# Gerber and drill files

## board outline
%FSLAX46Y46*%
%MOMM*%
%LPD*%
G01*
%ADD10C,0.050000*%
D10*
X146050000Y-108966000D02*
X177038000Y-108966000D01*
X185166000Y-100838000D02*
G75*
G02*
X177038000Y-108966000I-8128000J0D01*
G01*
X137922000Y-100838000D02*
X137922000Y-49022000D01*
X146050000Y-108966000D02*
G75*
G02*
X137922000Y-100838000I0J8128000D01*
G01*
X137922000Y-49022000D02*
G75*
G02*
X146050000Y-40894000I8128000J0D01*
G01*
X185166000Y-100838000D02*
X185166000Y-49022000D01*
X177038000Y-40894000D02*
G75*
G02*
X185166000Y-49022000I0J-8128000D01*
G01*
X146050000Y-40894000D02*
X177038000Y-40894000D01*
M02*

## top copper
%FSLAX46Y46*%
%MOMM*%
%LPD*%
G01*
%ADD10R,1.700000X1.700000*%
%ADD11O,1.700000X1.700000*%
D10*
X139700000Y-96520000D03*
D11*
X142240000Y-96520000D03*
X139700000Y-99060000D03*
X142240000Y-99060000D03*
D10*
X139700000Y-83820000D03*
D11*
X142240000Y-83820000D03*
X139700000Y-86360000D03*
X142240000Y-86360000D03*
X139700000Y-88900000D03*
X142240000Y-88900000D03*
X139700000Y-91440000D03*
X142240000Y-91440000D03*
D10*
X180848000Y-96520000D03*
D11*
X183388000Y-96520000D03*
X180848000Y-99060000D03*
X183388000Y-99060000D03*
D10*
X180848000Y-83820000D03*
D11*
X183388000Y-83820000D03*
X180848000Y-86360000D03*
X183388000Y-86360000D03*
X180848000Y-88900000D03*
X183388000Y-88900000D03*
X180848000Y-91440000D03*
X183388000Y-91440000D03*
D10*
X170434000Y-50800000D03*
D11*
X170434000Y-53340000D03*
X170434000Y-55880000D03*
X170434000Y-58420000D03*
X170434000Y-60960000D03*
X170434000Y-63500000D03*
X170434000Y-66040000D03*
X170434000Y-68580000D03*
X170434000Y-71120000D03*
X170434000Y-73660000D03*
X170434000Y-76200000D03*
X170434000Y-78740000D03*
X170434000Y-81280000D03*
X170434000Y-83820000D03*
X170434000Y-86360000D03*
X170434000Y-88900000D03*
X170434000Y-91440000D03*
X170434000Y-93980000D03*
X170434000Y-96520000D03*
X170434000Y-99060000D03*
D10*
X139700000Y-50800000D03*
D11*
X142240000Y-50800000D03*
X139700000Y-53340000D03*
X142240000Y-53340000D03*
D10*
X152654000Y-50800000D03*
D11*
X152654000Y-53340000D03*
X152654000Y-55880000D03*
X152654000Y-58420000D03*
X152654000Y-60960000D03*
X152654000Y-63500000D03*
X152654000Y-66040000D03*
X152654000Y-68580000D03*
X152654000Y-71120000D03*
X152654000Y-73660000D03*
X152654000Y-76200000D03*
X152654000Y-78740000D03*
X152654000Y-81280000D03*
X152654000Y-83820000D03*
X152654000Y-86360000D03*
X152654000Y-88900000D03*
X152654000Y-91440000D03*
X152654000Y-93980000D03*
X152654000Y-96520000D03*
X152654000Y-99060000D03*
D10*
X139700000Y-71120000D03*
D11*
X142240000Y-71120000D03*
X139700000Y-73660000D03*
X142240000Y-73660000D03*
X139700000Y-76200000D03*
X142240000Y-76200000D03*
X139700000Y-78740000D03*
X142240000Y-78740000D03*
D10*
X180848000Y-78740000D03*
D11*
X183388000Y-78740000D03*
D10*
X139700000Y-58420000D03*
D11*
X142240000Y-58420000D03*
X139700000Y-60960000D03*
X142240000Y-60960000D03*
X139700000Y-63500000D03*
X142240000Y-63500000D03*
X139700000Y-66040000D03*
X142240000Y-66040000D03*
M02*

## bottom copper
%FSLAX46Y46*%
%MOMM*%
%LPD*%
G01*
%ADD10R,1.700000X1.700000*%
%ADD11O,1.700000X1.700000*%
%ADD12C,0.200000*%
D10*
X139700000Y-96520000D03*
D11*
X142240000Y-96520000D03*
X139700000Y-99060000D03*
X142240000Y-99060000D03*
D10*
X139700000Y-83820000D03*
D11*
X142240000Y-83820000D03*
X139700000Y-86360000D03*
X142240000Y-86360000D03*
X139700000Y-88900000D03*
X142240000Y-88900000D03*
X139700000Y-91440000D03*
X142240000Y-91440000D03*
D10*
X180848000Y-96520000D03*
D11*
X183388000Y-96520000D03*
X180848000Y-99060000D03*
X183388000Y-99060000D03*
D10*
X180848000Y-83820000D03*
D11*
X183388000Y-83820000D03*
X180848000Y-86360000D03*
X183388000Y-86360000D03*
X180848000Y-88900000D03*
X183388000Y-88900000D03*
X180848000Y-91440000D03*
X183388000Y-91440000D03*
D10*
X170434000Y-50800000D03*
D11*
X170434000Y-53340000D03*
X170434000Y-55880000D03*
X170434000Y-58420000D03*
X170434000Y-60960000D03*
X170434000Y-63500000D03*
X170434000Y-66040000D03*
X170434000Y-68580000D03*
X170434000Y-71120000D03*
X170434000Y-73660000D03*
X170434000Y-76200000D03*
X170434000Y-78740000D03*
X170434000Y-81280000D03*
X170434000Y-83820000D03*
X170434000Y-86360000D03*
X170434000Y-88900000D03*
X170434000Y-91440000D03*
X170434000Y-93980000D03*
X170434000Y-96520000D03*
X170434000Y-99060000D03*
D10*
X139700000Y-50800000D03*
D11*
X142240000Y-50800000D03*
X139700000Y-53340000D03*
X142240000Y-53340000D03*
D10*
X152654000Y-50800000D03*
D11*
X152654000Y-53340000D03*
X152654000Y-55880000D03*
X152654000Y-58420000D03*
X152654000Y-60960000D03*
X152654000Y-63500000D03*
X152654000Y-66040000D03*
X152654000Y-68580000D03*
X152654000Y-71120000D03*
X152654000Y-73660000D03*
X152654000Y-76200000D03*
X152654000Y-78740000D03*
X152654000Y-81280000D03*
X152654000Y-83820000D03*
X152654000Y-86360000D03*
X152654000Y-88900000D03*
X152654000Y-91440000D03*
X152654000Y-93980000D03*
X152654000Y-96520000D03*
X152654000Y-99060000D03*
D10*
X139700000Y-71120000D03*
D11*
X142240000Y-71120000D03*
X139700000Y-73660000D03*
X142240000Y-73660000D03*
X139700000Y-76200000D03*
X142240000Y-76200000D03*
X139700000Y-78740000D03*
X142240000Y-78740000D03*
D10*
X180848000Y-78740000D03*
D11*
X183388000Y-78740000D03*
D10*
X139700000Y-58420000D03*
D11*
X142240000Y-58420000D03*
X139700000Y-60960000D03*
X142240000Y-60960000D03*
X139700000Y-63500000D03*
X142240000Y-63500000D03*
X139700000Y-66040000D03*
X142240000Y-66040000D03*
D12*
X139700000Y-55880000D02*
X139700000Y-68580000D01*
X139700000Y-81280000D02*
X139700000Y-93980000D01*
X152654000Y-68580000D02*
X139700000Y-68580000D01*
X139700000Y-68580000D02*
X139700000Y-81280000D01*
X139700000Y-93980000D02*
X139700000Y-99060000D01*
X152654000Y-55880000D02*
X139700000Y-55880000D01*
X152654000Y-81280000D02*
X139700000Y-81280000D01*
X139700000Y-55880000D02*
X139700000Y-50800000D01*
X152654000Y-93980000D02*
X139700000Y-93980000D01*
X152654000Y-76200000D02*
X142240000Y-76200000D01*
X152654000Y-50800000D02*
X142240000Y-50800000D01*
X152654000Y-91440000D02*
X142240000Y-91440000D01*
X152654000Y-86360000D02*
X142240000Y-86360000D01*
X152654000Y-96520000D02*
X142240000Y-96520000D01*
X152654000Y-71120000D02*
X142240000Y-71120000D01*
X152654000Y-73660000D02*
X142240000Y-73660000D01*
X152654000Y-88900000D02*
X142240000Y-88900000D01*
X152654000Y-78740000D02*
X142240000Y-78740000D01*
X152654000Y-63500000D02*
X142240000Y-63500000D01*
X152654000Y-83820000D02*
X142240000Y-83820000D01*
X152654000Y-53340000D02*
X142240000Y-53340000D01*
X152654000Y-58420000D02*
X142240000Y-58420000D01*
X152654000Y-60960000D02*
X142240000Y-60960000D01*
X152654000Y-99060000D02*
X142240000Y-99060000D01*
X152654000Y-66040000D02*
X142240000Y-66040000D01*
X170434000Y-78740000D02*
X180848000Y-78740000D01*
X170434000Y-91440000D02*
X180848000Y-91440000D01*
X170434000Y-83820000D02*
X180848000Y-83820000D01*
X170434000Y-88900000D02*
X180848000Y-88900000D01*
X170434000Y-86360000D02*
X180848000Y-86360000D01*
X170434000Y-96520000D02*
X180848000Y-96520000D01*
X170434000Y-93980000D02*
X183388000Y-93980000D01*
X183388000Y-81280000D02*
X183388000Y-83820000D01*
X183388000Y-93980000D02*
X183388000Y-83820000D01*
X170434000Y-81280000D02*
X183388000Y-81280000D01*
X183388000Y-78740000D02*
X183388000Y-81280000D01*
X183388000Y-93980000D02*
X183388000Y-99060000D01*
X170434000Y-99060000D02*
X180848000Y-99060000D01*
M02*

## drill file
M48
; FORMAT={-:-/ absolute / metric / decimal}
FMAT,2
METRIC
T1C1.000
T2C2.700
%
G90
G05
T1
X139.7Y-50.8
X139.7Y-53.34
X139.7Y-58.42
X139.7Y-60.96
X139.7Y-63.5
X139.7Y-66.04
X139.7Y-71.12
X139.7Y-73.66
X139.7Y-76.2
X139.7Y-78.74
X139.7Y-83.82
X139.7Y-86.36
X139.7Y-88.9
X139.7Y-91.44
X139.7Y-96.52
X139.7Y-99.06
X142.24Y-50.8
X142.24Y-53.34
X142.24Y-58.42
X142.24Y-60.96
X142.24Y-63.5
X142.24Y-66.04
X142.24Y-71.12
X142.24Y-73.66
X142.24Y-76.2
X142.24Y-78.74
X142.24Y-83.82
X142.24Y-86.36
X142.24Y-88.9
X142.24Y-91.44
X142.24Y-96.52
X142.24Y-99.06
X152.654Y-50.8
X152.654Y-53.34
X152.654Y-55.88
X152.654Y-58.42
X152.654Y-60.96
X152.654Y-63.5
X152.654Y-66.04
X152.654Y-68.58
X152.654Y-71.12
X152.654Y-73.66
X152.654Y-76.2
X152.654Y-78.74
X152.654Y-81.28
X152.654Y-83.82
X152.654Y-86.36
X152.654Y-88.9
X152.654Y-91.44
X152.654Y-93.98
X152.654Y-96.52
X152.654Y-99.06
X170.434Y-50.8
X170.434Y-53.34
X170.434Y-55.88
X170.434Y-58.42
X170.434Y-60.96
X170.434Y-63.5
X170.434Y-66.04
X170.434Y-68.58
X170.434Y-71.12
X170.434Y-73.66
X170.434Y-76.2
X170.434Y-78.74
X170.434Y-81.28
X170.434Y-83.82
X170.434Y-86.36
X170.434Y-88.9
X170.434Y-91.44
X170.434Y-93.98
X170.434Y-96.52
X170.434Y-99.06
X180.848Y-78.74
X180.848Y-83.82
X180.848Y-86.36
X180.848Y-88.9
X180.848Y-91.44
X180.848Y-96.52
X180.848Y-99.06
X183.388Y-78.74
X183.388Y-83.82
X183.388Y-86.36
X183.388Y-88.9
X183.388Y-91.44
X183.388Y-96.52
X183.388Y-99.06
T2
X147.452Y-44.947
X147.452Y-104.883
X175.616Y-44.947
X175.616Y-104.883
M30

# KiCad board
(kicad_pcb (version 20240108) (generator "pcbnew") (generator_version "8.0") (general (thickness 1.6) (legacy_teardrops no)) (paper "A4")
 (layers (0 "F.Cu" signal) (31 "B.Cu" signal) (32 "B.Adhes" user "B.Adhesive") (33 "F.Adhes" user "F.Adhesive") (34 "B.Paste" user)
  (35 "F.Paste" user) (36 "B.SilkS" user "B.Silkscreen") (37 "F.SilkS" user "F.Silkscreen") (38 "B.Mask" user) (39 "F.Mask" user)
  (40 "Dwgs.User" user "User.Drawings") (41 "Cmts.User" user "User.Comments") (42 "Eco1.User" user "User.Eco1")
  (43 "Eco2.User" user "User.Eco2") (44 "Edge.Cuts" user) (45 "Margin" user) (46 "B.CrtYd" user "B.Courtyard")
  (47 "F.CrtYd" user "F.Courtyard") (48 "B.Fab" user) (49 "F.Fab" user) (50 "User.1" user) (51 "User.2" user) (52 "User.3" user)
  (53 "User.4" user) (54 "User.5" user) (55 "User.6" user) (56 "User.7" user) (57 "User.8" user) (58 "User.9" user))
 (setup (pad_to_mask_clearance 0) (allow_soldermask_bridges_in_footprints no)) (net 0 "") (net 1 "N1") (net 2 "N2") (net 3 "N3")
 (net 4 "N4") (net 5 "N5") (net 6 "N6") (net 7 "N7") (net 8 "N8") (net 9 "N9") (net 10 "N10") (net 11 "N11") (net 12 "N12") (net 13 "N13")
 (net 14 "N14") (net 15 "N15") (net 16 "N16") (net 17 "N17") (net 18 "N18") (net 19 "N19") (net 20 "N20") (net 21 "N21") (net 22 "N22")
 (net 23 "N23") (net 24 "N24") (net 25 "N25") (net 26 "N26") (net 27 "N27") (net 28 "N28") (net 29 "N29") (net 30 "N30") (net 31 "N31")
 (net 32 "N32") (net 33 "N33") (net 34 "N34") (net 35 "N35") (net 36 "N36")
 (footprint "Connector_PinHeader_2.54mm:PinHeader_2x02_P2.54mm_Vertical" (layer "F.Cu") (at 139.7 96.52)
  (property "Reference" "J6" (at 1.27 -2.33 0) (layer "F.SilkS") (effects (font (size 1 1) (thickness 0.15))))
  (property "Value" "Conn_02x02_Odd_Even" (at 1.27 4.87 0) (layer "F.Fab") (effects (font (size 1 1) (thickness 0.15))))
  (pad "1" thru_hole rect (at 0 0) (size 1.7 1.7) (drill 1) (layers "*.Cu" "*.Mask") (remove_unused_layers no) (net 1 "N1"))
  (pad "2" thru_hole oval (at 2.54 0) (size 1.7 1.7) (drill 1) (layers "*.Cu" "*.Mask") (remove_unused_layers no) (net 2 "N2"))
  (pad "3" thru_hole oval (at 0 2.54) (size 1.7 1.7) (drill 1) (layers "*.Cu" "*.Mask") (remove_unused_layers no) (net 1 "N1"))
  (pad "4" thru_hole oval (at 2.54 2.54) (size 1.7 1.7) (drill 1) (layers "*.Cu" "*.Mask") (remove_unused_layers no) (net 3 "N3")))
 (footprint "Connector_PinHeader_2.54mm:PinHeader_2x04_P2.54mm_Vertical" (layer "F.Cu") (at 139.7 83.82)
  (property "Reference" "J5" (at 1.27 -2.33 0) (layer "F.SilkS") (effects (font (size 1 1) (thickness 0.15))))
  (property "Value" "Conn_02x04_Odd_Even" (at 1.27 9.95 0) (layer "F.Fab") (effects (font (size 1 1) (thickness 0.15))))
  (pad "1" thru_hole rect (at 0 0) (size 1.7 1.7) (drill 1) (layers "*.Cu" "*.Mask") (remove_unused_layers no) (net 1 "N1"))
  (pad "2" thru_hole oval (at 2.54 0) (size 1.7 1.7) (drill 1) (layers "*.Cu" "*.Mask") (remove_unused_layers no) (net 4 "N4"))
  (pad "3" thru_hole oval (at 0 2.54) (size 1.7 1.7) (drill 1) (layers "*.Cu" "*.Mask") (remove_unused_layers no) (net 1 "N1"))
  (pad "4" thru_hole oval (at 2.54 2.54) (size 1.7 1.7) (drill 1) (layers "*.Cu" "*.Mask") (remove_unused_layers no) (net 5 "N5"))
  (pad "5" thru_hole oval (at 0 5.08) (size 1.7 1.7) (drill 1) (layers "*.Cu" "*.Mask") (remove_unused_layers no) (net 1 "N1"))
  (pad "6" thru_hole oval (at 2.54 5.08) (size 1.7 1.7) (drill 1) (layers "*.Cu" "*.Mask") (remove_unused_layers no) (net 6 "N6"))
  (pad "7" thru_hole oval (at 0 7.62) (size 1.7 1.7) (drill 1) (layers "*.Cu" "*.Mask") (remove_unused_layers no) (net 1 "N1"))
  (pad "8" thru_hole oval (at 2.54 7.62) (size 1.7 1.7) (drill 1) (layers "*.Cu" "*.Mask") (remove_unused_layers no) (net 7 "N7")))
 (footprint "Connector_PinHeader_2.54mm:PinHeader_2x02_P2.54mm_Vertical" (layer "F.Cu") (at 180.848 96.52)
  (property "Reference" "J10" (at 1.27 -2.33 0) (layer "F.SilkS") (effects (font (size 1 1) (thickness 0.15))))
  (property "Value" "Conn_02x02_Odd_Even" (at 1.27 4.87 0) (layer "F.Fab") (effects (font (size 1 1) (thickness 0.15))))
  (pad "1" thru_hole rect (at 0 0) (size 1.7 1.7) (drill 1) (layers "*.Cu" "*.Mask") (remove_unused_layers no) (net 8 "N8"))
  (pad "2" thru_hole oval (at 2.54 0) (size 1.7 1.7) (drill 1) (layers "*.Cu" "*.Mask") (remove_unused_layers no) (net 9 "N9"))
  (pad "3" thru_hole oval (at 0 2.54) (size 1.7 1.7) (drill 1) (layers "*.Cu" "*.Mask") (remove_unused_layers no) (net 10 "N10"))
  (pad "4" thru_hole oval (at 2.54 2.54) (size 1.7 1.7) (drill 1) (layers "*.Cu" "*.Mask") (remove_unused_layers no) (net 9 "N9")))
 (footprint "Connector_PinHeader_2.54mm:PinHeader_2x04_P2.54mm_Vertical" (layer "F.Cu") (at 180.848 83.82)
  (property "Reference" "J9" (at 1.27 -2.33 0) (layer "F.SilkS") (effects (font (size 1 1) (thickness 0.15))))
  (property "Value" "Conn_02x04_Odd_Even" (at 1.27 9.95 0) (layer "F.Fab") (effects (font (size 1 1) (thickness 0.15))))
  (pad "1" thru_hole rect (at 0 0) (size 1.7 1.7) (drill 1) (layers "*.Cu" "*.Mask") (remove_unused_layers no) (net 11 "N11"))
  (pad "2" thru_hole oval (at 2.54 0) (size 1.7 1.7) (drill 1) (layers "*.Cu" "*.Mask") (remove_unused_layers no) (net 9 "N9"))
  (pad "3" thru_hole oval (at 0 2.54) (size 1.7 1.7) (drill 1) (layers "*.Cu" "*.Mask") (remove_unused_layers no) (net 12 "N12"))
  (pad "4" thru_hole oval (at 2.54 2.54) (size 1.7 1.7) (drill 1) (layers "*.Cu" "*.Mask") (remove_unused_layers no) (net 9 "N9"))
  (pad "5" thru_hole oval (at 0 5.08) (size 1.7 1.7) (drill 1) (layers "*.Cu" "*.Mask") (remove_unused_layers no) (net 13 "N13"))
  (pad "6" thru_hole oval (at 2.54 5.08) (size 1.7 1.7) (drill 1) (layers "*.Cu" "*.Mask") (remove_unused_layers no) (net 9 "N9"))
  (pad "7" thru_hole oval (at 0 7.62) (size 1.7 1.7) (drill 1) (layers "*.Cu" "*.Mask") (remove_unused_layers no) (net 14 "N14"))
  (pad "8" thru_hole oval (at 2.54 7.62) (size 1.7 1.7) (drill 1) (layers "*.Cu" "*.Mask") (remove_unused_layers no) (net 9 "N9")))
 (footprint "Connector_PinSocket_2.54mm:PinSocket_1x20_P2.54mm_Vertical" (layer "F.Cu") (at 170.434 50.8)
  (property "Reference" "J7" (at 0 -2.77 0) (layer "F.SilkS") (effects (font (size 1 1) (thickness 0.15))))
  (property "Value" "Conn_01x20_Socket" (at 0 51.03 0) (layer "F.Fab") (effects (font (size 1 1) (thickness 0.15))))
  (pad "1" thru_hole rect (at 0 0) (size 1.7 1.7) (drill 1) (layers "*.Cu" "*.Mask") (remove_unused_layers no) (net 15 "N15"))
  (pad "2" thru_hole oval (at 0 2.54) (size 1.7 1.7) (drill 1) (layers "*.Cu" "*.Mask") (remove_unused_layers no) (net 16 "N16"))
  (pad "3" thru_hole oval (at 0 5.08) (size 1.7 1.7) (drill 1) (layers "*.Cu" "*.Mask") (remove_unused_layers no) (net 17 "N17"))
  (pad "4" thru_hole oval (at 0 7.62) (size 1.7 1.7) (drill 1) (layers "*.Cu" "*.Mask") (remove_unused_layers no) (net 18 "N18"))
  (pad "5" thru_hole oval (at 0 10.16) (size 1.7 1.7) (drill 1) (layers "*.Cu" "*.Mask") (remove_unused_layers no) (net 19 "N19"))
  (pad "6" thru_hole oval (at 0 12.7) (size 1.7 1.7) (drill 1) (layers "*.Cu" "*.Mask") (remove_unused_layers no) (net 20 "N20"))
  (pad "7" thru_hole oval (at 0 15.24) (size 1.7 1.7) (drill 1) (layers "*.Cu" "*.Mask") (remove_unused_layers no) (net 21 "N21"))
  (pad "8" thru_hole oval (at 0 17.78) (size 1.7 1.7) (drill 1) (layers "*.Cu" "*.Mask") (remove_unused_layers no) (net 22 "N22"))
  (pad "9" thru_hole oval (at 0 20.32) (size 1.7 1.7) (drill 1) (layers "*.Cu" "*.Mask") (remove_unused_layers no) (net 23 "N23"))
  (pad "10" thru_hole oval (at 0 22.86) (size 1.7 1.7) (drill 1) (layers "*.Cu" "*.Mask") (remove_unused_layers no) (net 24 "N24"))
  (pad "11" thru_hole oval (at 0 25.4) (size 1.7 1.7) (drill 1) (layers "*.Cu" "*.Mask") (remove_unused_layers no) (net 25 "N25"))
  (pad "12" thru_hole oval (at 0 27.94) (size 1.7 1.7) (drill 1) (layers "*.Cu" "*.Mask") (remove_unused_layers no) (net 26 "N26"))
  (pad "13" thru_hole oval (at 0 30.48) (size 1.7 1.7) (drill 1) (layers "*.Cu" "*.Mask") (remove_unused_layers no) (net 9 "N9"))
  (pad "14" thru_hole oval (at 0 33.02) (size 1.7 1.7) (drill 1) (layers "*.Cu" "*.Mask") (remove_unused_layers no) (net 11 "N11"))
  (pad "15" thru_hole oval (at 0 35.56) (size 1.7 1.7) (drill 1) (layers "*.Cu" "*.Mask") (remove_unused_layers no) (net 12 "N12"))
  (pad "16" thru_hole oval (at 0 38.1) (size 1.7 1.7) (drill 1) (layers "*.Cu" "*.Mask") (remove_unused_layers no) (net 13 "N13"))
  (pad "17" thru_hole oval (at 0 40.64) (size 1.7 1.7) (drill 1) (layers "*.Cu" "*.Mask") (remove_unused_layers no) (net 14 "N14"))
  (pad "18" thru_hole oval (at 0 43.18) (size 1.7 1.7) (drill 1) (layers "*.Cu" "*.Mask") (remove_unused_layers no) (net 9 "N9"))
  (pad "19" thru_hole oval (at 0 45.72) (size 1.7 1.7) (drill 1) (layers "*.Cu" "*.Mask") (remove_unused_layers no) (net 8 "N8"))
  (pad "20" thru_hole oval (at 0 48.26) (size 1.7 1.7) (drill 1) (layers "*.Cu" "*.Mask") (remove_unused_layers no) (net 10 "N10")))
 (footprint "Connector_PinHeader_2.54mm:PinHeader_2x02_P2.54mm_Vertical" (layer "F.Cu") (at 139.7 50.8)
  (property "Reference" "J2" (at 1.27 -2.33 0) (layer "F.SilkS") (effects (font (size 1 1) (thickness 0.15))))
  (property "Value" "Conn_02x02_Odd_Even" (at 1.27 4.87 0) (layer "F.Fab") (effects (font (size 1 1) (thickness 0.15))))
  (pad "1" thru_hole rect (at 0 0) (size 1.7 1.7) (drill 1) (layers "*.Cu" "*.Mask") (remove_unused_layers no) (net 1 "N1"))
  (pad "2" thru_hole oval (at 2.54 0) (size 1.7 1.7) (drill 1) (layers "*.Cu" "*.Mask") (remove_unused_layers no) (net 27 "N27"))
  (pad "3" thru_hole oval (at 0 2.54) (size 1.7 1.7) (drill 1) (layers "*.Cu" "*.Mask") (remove_unused_layers no) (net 1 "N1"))
  (pad "4" thru_hole oval (at 2.54 2.54) (size 1.7 1.7) (drill 1) (layers "*.Cu" "*.Mask") (remove_unused_layers no) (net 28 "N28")))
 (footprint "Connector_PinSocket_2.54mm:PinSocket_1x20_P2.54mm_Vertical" (layer "F.Cu") (at 152.654 50.8)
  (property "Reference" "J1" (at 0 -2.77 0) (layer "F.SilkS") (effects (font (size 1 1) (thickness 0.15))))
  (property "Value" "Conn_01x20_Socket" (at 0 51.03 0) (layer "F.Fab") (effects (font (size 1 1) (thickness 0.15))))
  (pad "1" thru_hole rect (at 0 0) (size 1.7 1.7) (drill 1) (layers "*.Cu" "*.Mask") (remove_unused_layers no) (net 27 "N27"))
  (pad "2" thru_hole oval (at 0 2.54) (size 1.7 1.7) (drill 1) (layers "*.Cu" "*.Mask") (remove_unused_layers no) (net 28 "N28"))
  (pad "3" thru_hole oval (at 0 5.08) (size 1.7 1.7) (drill 1) (layers "*.Cu" "*.Mask") (remove_unused_layers no) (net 1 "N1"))
  (pad "4" thru_hole oval (at 0 7.62) (size 1.7 1.7) (drill 1) (layers "*.Cu" "*.Mask") (remove_unused_layers no) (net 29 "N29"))
  (pad "5" thru_hole oval (at 0 10.16) (size 1.7 1.7) (drill 1) (layers "*.Cu" "*.Mask") (remove_unused_layers no) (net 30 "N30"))
  (pad "6" thru_hole oval (at 0 12.7) (size 1.7 1.7) (drill 1) (layers "*.Cu" "*.Mask") (remove_unused_layers no) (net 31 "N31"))
  (pad "7" thru_hole oval (at 0 15.24) (size 1.7 1.7) (drill 1) (layers "*.Cu" "*.Mask") (remove_unused_layers no) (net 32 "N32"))
  (pad "8" thru_hole oval (at 0 17.78) (size 1.7 1.7) (drill 1) (layers "*.Cu" "*.Mask") (remove_unused_layers no) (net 1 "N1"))
  (pad "9" thru_hole oval (at 0 20.32) (size 1.7 1.7) (drill 1) (layers "*.Cu" "*.Mask") (remove_unused_layers no) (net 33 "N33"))
  (pad "10" thru_hole oval (at 0 22.86) (size 1.7 1.7) (drill 1) (layers "*.Cu" "*.Mask") (remove_unused_layers no) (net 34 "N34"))
  (pad "11" thru_hole oval (at 0 25.4) (size 1.7 1.7) (drill 1) (layers "*.Cu" "*.Mask") (remove_unused_layers no) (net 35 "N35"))
  (pad "12" thru_hole oval (at 0 27.94) (size 1.7 1.7) (drill 1) (layers "*.Cu" "*.Mask") (remove_unused_layers no) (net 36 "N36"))
  (pad "13" thru_hole oval (at 0 30.48) (size 1.7 1.7) (drill 1) (layers "*.Cu" "*.Mask") (remove_unused_layers no) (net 1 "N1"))
  (pad "14" thru_hole oval (at 0 33.02) (size 1.7 1.7) (drill 1) (layers "*.Cu" "*.Mask") (remove_unused_layers no) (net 4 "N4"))
  (pad "15" thru_hole oval (at 0 35.56) (size 1.7 1.7) (drill 1) (layers "*.Cu" "*.Mask") (remove_unused_layers no) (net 5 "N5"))
  (pad "16" thru_hole oval (at 0 38.1) (size 1.7 1.7) (drill 1) (layers "*.Cu" "*.Mask") (remove_unused_layers no) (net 6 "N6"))
  (pad "17" thru_hole oval (at 0 40.64) (size 1.7 1.7) (drill 1) (layers "*.Cu" "*.Mask") (remove_unused_layers no) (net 7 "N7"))
  (pad "18" thru_hole oval (at 0 43.18) (size 1.7 1.7) (drill 1) (layers "*.Cu" "*.Mask") (remove_unused_layers no) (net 1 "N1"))
  (pad "19" thru_hole oval (at 0 45.72) (size 1.7 1.7) (drill 1) (layers "*.Cu" "*.Mask") (remove_unused_layers no) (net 2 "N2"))
  (pad "20" thru_hole oval (at 0 48.26) (size 1.7 1.7) (drill 1) (layers "*.Cu" "*.Mask") (remove_unused_layers no) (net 3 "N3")))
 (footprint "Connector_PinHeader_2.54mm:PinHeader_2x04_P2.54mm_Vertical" (layer "F.Cu") (at 139.7 71.12)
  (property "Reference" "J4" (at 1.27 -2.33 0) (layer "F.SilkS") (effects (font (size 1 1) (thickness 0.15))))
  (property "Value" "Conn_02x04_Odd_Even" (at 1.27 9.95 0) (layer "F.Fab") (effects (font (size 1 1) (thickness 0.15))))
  (pad "1" thru_hole rect (at 0 0) (size 1.7 1.7) (drill 1) (layers "*.Cu" "*.Mask") (remove_unused_layers no) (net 1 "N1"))
  (pad "2" thru_hole oval (at 2.54 0) (size 1.7 1.7) (drill 1) (layers "*.Cu" "*.Mask") (remove_unused_layers no) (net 33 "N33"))
  (pad "3" thru_hole oval (at 0 2.54) (size 1.7 1.7) (drill 1) (layers "*.Cu" "*.Mask") (remove_unused_layers no) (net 1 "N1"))
  (pad "4" thru_hole oval (at 2.54 2.54) (size 1.7 1.7) (drill 1) (layers "*.Cu" "*.Mask") (remove_unused_layers no) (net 34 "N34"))
  (pad "5" thru_hole oval (at 0 5.08) (size 1.7 1.7) (drill 1) (layers "*.Cu" "*.Mask") (remove_unused_layers no) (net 1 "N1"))
  (pad "6" thru_hole oval (at 2.54 5.08) (size 1.7 1.7) (drill 1) (layers "*.Cu" "*.Mask") (remove_unused_layers no) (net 35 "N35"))
  (pad "7" thru_hole oval (at 0 7.62) (size 1.7 1.7) (drill 1) (layers "*.Cu" "*.Mask") (remove_unused_layers no) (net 1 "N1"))
  (pad "8" thru_hole oval (at 2.54 7.62) (size 1.7 1.7) (drill 1) (layers "*.Cu" "*.Mask") (remove_unused_layers no) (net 36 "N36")))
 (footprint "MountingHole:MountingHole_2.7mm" (layer "F.Cu") (at 175.616 104.883)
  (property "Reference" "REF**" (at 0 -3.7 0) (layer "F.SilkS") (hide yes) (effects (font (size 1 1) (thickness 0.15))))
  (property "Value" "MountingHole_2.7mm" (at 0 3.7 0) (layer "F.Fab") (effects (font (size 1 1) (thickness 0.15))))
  (pad "" np_thru_hole circle (at 0 0) (size 2.7 2.7) (drill 2.7) (layers "*.Cu" "*.Mask")))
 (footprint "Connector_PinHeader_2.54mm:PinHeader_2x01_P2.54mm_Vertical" (layer "F.Cu") (at 180.848 78.74)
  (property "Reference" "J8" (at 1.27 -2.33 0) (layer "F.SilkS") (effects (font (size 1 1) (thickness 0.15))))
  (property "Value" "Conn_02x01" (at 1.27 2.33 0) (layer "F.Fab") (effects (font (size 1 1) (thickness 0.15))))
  (pad "1" thru_hole rect (at 0 0) (size 1.7 1.7) (drill 1) (layers "*.Cu" "*.Mask") (remove_unused_layers no) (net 26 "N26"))
  (pad "2" thru_hole oval (at 2.54 0) (size 1.7 1.7) (drill 1) (layers "*.Cu" "*.Mask") (remove_unused_layers no) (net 9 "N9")))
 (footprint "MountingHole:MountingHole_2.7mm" (layer "F.Cu") (at 147.452 104.883)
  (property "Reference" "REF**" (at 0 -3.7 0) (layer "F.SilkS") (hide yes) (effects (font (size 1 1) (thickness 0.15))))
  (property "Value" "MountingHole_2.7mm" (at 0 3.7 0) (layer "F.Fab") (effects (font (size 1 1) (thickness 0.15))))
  (pad "" np_thru_hole circle (at 0 0) (size 2.7 2.7) (drill 2.7) (layers "*.Cu" "*.Mask")))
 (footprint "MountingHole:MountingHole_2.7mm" (layer "F.Cu") (at 147.452 44.947)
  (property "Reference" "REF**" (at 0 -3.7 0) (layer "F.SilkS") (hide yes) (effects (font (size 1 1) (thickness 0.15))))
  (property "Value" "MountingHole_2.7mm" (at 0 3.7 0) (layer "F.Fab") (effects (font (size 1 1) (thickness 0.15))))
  (pad "" np_thru_hole circle (at 0 0) (size 2.7 2.7) (drill 2.7) (layers "*.Cu" "*.Mask")))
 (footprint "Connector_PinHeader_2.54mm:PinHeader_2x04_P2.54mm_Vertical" (layer "F.Cu") (at 139.7 58.42)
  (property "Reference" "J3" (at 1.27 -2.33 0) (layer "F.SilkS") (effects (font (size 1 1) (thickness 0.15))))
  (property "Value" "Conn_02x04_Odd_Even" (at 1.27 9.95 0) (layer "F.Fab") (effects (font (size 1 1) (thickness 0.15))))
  (pad "1" thru_hole rect (at 0 0) (size 1.7 1.7) (drill 1) (layers "*.Cu" "*.Mask") (remove_unused_layers no) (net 1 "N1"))
  (pad "2" thru_hole oval (at 2.54 0) (size 1.7 1.7) (drill 1) (layers "*.Cu" "*.Mask") (remove_unused_layers no) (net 29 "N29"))
  (pad "3" thru_hole oval (at 0 2.54) (size 1.7 1.7) (drill 1) (layers "*.Cu" "*.Mask") (remove_unused_layers no) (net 1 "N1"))
  (pad "4" thru_hole oval (at 2.54 2.54) (size 1.7 1.7) (drill 1) (layers "*.Cu" "*.Mask") (remove_unused_layers no) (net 30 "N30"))
  (pad "5" thru_hole oval (at 0 5.08) (size 1.7 1.7) (drill 1) (layers "*.Cu" "*.Mask") (remove_unused_layers no) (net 1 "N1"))
  (pad "6" thru_hole oval (at 2.54 5.08) (size 1.7 1.7) (drill 1) (layers "*.Cu" "*.Mask") (remove_unused_layers no) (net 31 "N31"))
  (pad "7" thru_hole oval (at 0 7.62) (size 1.7 1.7) (drill 1) (layers "*.Cu" "*.Mask") (remove_unused_layers no) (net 1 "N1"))
  (pad "8" thru_hole oval (at 2.54 7.62) (size 1.7 1.7) (drill 1) (layers "*.Cu" "*.Mask") (remove_unused_layers no) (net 32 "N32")))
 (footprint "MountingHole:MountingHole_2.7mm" (layer "F.Cu") (at 175.616 44.947)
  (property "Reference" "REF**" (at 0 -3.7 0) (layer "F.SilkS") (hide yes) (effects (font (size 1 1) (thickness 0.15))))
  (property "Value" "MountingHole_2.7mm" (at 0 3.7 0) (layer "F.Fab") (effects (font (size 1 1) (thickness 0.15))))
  (pad "" np_thru_hole circle (at 0 0) (size 2.7 2.7) (drill 2.7) (layers "*.Cu" "*.Mask")))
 (gr_line (start 146.05 108.966) (end 177.038 108.966) (stroke (width 0.05) (type default)) (layer "Edge.Cuts"))
 (gr_arc (start 185.166 100.838) (mid 182.785364 106.585364) (end 177.038 108.966) (stroke (width 0.05) (type default)) (layer "Edge.Cuts"))
 (gr_line (start 137.922 100.838) (end 137.922 49.022) (stroke (width 0.05) (type default)) (layer "Edge.Cuts"))
 (gr_arc (start 146.05 108.966) (mid 140.302636 106.585364) (end 137.922 100.838) (stroke (width 0.05) (type default)) (layer "Edge.Cuts"))
 (gr_arc (start 137.922 49.022) (mid 140.302636 43.274636) (end 146.05 40.894) (stroke (width 0.05) (type default)) (layer "Edge.Cuts"))
 (gr_line (start 185.166 100.838) (end 185.166 49.022) (stroke (width 0.05) (type default)) (layer "Edge.Cuts"))
 (gr_arc (start 177.038 40.894) (mid 182.785364 43.274636) (end 185.166 49.022) (stroke (width 0.05) (type default)) (layer "Edge.Cuts"))
 (gr_line (start 146.05 40.894) (end 177.038 40.894) (stroke (width 0.05) (type default)) (layer "Edge.Cuts"))
 (segment (start 139.7 55.88) (end 139.7 68.58) (width 0.2) (layer "B.Cu") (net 1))
 (segment (start 139.7 81.28) (end 139.7 93.98) (width 0.2) (layer "B.Cu") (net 1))
 (segment (start 152.654 68.58) (end 139.7 68.58) (width 0.2) (layer "B.Cu") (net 1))
 (segment (start 139.7 68.58) (end 139.7 81.28) (width 0.2) (layer "B.Cu") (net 1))
 (segment (start 139.7 93.98) (end 139.7 99.06) (width 0.2) (layer "B.Cu") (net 1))
 (segment (start 152.654 55.88) (end 139.7 55.88) (width 0.2) (layer "B.Cu") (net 1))
 (segment (start 152.654 81.28) (end 139.7 81.28) (width 0.2) (layer "B.Cu") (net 1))
 (segment (start 139.7 55.88) (end 139.7 50.8) (width 0.2) (layer "B.Cu") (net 1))
 (segment (start 152.654 93.98) (end 139.7 93.98) (width 0.2) (layer "B.Cu") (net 1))
 (segment (start 152.654 76.2) (end 142.24 76.2) (width 0.2) (layer "B.Cu") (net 35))
 (segment (start 152.654 50.8) (end 142.24 50.8) (width 0.2) (layer "B.Cu") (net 27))
 (segment (start 152.654 91.44) (end 142.24 91.44) (width 0.2) (layer "B.Cu") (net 7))
 (segment (start 152.654 86.36) (end 142.24 86.36) (width 0.2) (layer "B.Cu") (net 5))
 (segment (start 152.654 96.52) (end 142.24 96.52) (width 0.2) (layer "B.Cu") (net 2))
 (segment (start 152.654 71.12) (end 142.24 71.12) (width 0.2) (layer "B.Cu") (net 33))
 (segment (start 152.654 73.66) (end 142.24 73.66) (width 0.2) (layer "B.Cu") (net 34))
 (segment (start 152.654 88.9) (end 142.24 88.9) (width 0.2) (layer "B.Cu") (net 6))
 (segment (start 152.654 78.74) (end 142.24 78.74) (width 0.2) (layer "B.Cu") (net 36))
 (segment (start 152.654 63.5) (end 142.24 63.5) (width 0.2) (layer "B.Cu") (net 31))
 (segment (start 152.654 83.82) (end 142.24 83.82) (width 0.2) (layer "B.Cu") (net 4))
 (segment (start 152.654 53.34) (end 142.24 53.34) (width 0.2) (layer "B.Cu") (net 28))
 (segment (start 152.654 58.42) (end 142.24 58.42) (width 0.2) (layer "B.Cu") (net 29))
 (segment (start 152.654 60.96) (end 142.24 60.96) (width 0.2) (layer "B.Cu") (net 30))
 (segment (start 152.654 99.06) (end 142.24 99.06) (width 0.2) (layer "B.Cu") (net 3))
 (segment (start 152.654 66.04) (end 142.24 66.04) (width 0.2) (layer "B.Cu") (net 32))
 (segment (start 170.434 78.74) (end 180.848 78.74) (width 0.2) (layer "B.Cu") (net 26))
 (segment (start 170.434 91.44) (end 180.848 91.44) (width 0.2) (layer "B.Cu") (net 14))
 (segment (start 170.434 83.82) (end 180.848 83.82) (width 0.2) (layer "B.Cu") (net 11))
 (segment (start 170.434 88.9) (end 180.848 88.9) (width 0.2) (layer "B.Cu") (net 13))
 (segment (start 170.434 86.36) (end 180.848 86.36) (width 0.2) (layer "B.Cu") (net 12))
 (segment (start 170.434 96.52) (end 180.848 96.52) (width 0.2) (layer "B.Cu") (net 8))
 (segment (start 170.434 93.98) (end 183.388 93.98) (width 0.2) (layer "B.Cu") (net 9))
 (segment (start 183.388 81.28) (end 183.388 83.82) (width 0.2) (layer "B.Cu") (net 9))
 (segment (start 183.388 93.98) (end 183.388 83.82) (width 0.2) (layer "B.Cu") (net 9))
 (segment (start 170.434 81.28) (end 183.388 81.28) (width 0.2) (layer "B.Cu") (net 9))
 (segment (start 183.388 78.74) (end 183.388 81.28) (width 0.2) (layer "B.Cu") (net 9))
 (segment (start 183.388 93.98) (end 183.388 99.06) (width 0.2) (layer "B.Cu") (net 9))
 (segment (start 170.434 99.06) (end 180.848 99.06) (width 0.2) (layer "B.Cu") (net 10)))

